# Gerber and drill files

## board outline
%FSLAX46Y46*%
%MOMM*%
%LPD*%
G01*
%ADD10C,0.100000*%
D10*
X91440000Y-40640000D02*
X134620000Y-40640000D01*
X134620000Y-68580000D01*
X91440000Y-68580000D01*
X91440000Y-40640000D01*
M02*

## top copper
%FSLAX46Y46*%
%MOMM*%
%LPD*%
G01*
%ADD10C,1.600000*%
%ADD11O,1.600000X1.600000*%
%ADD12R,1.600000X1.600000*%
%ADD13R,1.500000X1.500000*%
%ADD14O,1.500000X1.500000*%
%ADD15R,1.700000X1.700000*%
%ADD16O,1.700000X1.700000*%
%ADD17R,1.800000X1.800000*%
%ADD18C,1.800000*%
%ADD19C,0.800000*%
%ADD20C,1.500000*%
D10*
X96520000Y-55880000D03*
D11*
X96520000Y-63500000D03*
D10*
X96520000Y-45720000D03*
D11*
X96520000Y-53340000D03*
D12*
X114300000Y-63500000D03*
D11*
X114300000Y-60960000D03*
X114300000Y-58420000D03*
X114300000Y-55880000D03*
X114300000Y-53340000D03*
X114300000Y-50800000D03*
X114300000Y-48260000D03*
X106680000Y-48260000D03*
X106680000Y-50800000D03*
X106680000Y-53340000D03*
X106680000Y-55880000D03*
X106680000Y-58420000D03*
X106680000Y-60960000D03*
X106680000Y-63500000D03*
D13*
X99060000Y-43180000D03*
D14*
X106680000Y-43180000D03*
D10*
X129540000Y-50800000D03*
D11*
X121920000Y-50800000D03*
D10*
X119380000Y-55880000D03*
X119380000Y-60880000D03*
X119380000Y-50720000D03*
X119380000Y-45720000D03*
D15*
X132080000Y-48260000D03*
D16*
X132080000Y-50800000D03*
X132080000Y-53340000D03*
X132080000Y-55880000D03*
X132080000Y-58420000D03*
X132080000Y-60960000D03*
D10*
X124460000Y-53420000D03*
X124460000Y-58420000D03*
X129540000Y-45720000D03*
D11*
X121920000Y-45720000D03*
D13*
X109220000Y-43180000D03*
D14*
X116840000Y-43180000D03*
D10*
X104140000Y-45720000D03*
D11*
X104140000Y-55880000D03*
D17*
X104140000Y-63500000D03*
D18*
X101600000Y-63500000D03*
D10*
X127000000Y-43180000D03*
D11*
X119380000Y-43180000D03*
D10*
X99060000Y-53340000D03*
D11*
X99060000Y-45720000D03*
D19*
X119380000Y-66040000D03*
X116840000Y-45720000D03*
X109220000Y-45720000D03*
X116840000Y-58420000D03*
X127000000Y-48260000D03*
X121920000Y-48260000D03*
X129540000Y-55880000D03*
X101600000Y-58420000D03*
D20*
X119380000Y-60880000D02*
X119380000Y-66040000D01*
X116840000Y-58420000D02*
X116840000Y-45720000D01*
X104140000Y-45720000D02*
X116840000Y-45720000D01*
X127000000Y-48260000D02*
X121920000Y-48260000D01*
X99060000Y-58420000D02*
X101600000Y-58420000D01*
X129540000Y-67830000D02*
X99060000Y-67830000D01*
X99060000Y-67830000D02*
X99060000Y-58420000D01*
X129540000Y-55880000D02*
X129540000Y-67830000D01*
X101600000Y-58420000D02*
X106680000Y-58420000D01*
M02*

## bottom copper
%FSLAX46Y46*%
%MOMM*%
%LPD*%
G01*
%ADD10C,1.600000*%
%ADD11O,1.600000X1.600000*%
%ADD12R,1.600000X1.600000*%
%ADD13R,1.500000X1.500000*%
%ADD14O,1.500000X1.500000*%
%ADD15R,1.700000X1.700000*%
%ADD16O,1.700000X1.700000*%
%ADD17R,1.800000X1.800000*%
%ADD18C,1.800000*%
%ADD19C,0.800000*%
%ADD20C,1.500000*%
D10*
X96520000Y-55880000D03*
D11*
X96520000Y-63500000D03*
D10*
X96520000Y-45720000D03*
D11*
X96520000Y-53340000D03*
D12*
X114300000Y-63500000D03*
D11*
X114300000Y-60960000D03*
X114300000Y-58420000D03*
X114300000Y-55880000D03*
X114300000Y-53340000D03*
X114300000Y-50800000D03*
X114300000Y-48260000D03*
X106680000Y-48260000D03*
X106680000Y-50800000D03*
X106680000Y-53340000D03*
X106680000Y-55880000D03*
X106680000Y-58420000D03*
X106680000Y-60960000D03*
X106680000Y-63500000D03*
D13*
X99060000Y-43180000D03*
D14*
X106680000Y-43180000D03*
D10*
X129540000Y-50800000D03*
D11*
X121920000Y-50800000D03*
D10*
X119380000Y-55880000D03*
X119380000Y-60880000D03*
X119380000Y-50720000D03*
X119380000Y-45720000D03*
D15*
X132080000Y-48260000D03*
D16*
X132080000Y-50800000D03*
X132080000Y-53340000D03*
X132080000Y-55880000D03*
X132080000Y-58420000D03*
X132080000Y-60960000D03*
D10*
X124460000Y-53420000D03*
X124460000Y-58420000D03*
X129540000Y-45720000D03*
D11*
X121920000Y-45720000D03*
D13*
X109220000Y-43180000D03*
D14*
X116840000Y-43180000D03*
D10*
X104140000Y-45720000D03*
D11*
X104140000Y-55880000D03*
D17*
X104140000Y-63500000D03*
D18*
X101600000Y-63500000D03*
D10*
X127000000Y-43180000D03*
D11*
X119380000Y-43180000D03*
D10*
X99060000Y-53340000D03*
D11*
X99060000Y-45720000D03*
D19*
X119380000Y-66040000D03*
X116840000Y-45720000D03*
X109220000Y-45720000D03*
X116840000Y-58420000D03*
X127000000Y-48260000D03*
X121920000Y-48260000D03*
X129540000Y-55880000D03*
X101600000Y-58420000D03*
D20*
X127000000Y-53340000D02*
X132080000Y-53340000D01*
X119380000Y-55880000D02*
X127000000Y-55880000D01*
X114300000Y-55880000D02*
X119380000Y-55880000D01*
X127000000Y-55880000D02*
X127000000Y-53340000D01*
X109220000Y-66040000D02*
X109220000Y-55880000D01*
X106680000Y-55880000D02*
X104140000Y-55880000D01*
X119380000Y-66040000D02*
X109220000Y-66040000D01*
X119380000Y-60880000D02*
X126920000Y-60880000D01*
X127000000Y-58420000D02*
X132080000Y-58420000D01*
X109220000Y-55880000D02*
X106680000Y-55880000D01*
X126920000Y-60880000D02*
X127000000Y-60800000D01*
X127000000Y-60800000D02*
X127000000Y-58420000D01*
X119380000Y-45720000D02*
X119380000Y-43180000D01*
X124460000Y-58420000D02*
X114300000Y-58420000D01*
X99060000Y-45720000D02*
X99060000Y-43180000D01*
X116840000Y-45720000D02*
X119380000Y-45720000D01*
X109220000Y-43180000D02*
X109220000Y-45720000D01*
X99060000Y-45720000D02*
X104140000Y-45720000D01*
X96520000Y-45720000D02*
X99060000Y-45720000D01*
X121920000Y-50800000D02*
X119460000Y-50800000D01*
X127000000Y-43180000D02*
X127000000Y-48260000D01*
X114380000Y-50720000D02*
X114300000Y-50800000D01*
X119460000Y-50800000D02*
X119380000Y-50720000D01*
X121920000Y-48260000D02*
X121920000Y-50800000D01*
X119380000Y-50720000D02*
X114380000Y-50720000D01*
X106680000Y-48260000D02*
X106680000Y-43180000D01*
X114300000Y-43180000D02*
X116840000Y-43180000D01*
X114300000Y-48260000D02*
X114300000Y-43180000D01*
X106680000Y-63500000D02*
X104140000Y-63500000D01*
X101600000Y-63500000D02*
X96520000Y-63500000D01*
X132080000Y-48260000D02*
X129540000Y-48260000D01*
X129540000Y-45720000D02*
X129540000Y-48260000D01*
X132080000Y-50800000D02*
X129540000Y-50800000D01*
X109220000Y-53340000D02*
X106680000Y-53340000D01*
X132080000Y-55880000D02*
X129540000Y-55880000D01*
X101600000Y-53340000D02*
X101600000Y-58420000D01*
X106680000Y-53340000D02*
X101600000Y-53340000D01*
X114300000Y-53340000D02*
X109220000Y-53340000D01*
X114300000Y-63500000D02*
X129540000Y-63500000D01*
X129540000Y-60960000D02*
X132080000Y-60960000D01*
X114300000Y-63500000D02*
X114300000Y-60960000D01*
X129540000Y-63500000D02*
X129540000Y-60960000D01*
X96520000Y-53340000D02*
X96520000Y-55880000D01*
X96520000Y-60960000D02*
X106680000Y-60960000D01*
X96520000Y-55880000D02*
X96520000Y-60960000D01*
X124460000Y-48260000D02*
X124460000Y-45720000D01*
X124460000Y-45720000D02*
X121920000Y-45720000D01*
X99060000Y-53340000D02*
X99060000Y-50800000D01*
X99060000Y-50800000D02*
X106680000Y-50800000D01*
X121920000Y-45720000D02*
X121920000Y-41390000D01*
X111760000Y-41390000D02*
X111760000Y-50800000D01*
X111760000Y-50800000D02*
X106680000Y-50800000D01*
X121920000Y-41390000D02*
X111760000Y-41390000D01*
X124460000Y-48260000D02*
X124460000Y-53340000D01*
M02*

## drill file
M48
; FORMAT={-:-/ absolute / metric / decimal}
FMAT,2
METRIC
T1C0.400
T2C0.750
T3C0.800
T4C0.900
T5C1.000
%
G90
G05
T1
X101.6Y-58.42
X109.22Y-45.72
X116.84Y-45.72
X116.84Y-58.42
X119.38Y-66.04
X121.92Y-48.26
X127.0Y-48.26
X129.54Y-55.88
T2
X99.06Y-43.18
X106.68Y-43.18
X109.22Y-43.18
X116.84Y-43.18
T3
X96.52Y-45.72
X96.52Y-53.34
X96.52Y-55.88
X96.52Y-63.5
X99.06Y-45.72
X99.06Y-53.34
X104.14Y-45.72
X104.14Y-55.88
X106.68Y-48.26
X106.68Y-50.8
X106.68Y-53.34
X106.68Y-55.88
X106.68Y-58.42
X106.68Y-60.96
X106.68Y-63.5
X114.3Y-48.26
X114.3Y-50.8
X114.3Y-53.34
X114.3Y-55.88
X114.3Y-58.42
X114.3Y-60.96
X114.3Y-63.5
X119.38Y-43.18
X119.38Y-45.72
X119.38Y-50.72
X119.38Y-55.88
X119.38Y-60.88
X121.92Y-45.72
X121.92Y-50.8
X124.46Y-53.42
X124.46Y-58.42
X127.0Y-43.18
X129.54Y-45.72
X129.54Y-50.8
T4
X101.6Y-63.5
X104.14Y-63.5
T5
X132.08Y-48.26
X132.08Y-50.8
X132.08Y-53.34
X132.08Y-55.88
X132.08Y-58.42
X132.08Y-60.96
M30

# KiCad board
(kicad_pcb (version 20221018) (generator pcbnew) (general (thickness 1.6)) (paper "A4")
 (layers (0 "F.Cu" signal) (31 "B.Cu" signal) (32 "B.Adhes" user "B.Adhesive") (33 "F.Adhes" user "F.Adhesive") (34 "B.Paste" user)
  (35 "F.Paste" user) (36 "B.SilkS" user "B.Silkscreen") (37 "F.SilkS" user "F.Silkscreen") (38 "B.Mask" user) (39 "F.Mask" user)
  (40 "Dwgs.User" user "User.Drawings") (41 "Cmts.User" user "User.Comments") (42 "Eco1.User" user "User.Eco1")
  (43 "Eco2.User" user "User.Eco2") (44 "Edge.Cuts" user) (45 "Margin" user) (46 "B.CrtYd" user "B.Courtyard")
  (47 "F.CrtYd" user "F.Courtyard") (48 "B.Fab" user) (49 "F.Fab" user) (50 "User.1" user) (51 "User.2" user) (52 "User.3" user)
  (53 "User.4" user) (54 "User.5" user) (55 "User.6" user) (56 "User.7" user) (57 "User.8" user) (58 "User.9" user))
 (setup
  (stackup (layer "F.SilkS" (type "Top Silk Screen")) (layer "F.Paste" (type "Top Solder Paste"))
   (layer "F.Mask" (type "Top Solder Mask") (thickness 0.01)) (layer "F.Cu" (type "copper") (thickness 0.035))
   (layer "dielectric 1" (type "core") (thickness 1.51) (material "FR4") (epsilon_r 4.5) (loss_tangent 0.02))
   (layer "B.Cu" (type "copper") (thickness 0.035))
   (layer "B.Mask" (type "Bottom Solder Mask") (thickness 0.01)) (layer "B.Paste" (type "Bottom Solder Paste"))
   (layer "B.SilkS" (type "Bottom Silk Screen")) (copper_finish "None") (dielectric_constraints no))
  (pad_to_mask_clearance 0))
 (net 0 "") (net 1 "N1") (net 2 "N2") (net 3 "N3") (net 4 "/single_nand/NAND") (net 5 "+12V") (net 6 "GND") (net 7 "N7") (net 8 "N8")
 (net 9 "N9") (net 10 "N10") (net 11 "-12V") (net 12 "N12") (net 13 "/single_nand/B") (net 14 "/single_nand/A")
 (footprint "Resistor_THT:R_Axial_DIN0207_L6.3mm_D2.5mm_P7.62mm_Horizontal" (layer "F.Cu") (at 96.52 55.88 -90)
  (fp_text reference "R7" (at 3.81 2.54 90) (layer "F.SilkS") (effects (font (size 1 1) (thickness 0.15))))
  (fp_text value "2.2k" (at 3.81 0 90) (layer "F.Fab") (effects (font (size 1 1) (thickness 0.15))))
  (pad "1" thru_hole circle (at 0 0 270) (size 1.6 1.6) (drill 0.8) (layers "*.Cu" "*.Mask") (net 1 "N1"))
  (pad "2" thru_hole oval (at 7.62 0 270) (size 1.6 1.6) (drill 0.8) (layers "*.Cu" "*.Mask") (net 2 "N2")))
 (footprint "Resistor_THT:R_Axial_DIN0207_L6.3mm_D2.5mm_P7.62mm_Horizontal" (layer "F.Cu") (at 96.52 45.72 -90)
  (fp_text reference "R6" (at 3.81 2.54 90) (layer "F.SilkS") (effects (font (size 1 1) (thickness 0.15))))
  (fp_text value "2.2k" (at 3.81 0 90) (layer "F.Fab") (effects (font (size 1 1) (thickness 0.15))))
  (pad "1" thru_hole circle (at 0 0 270) (size 1.6 1.6) (drill 0.8) (layers "*.Cu" "*.Mask") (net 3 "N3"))
  (pad "2" thru_hole oval (at 7.62 0 270) (size 1.6 1.6) (drill 0.8) (layers "*.Cu" "*.Mask") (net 1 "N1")))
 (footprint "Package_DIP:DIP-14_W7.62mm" (layer "F.Cu") (at 114.3 63.5 180)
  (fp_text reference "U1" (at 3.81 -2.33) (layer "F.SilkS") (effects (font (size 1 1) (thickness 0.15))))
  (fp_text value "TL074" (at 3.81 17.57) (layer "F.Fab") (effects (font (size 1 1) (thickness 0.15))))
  (pad "1" thru_hole rect (at 0 0 180) (size 1.6 1.6) (drill 0.8) (layers "*.Cu" "*.Mask") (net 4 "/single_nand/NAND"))
  (pad "2" thru_hole oval (at 0 2.54 180) (size 1.6 1.6) (drill 0.8) (layers "*.Cu" "*.Mask") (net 4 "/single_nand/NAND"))
  (pad "3" thru_hole oval (at 0 5.08 180) (size 1.6 1.6) (drill 0.8) (layers "*.Cu" "*.Mask") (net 3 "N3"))
  (pad "4" thru_hole oval (at 0 7.62 180) (size 1.6 1.6) (drill 0.8) (layers "*.Cu" "*.Mask") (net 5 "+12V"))
  (pad "5" thru_hole oval (at 0 10.16 180) (size 1.6 1.6) (drill 0.8) (layers "*.Cu" "*.Mask") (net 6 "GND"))
  (pad "6" thru_hole oval (at 0 12.7 180) (size 1.6 1.6) (drill 0.8) (layers "*.Cu" "*.Mask") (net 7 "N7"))
  (pad "7" thru_hole oval (at 0 15.24 180) (size 1.6 1.6) (drill 0.8) (layers "*.Cu" "*.Mask") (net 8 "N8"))
  (pad "8" thru_hole oval (at 7.62 15.24 180) (size 1.6 1.6) (drill 0.8) (layers "*.Cu" "*.Mask") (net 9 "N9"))
  (pad "9" thru_hole oval (at 7.62 12.7 180) (size 1.6 1.6) (drill 0.8) (layers "*.Cu" "*.Mask") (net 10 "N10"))
  (pad "10" thru_hole oval (at 7.62 10.16 180) (size 1.6 1.6) (drill 0.8) (layers "*.Cu" "*.Mask") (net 6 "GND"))
  (pad "11" thru_hole oval (at 7.62 7.62 180) (size 1.6 1.6) (drill 0.8) (layers "*.Cu" "*.Mask") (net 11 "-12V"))
  (pad "12" thru_hole oval (at 7.62 5.08 180) (size 1.6 1.6) (drill 0.8) (layers "*.Cu" "*.Mask") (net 6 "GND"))
  (pad "13" thru_hole oval (at 7.62 2.54 180) (size 1.6 1.6) (drill 0.8) (layers "*.Cu" "*.Mask") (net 1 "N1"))
  (pad "14" thru_hole oval (at 7.62 0 180) (size 1.6 1.6) (drill 0.8) (layers "*.Cu" "*.Mask") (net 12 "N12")))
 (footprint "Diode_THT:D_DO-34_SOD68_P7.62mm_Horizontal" (layer "F.Cu") (at 99.06 43.18)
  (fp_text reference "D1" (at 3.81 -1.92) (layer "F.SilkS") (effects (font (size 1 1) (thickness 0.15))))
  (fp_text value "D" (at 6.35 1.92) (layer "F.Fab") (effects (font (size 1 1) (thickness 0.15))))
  (pad "1" thru_hole rect (at 0 0) (size 1.5 1.5) (drill 0.75) (layers "*.Cu" "*.Mask") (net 3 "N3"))
  (pad "2" thru_hole oval (at 7.62 0) (size 1.5 1.5) (drill 0.75) (layers "*.Cu" "*.Mask") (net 9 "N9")))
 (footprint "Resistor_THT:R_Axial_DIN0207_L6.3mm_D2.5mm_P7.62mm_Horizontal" (layer "F.Cu") (at 129.54 50.8 180)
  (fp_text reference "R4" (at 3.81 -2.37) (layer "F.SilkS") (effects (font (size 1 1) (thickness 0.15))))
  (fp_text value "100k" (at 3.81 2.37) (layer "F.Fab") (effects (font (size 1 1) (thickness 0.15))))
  (pad "1" thru_hole circle (at 0 0 180) (size 1.6 1.6) (drill 0.8) (layers "*.Cu" "*.Mask") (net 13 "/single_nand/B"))
  (pad "2" thru_hole oval (at 7.62 0 180) (size 1.6 1.6) (drill 0.8) (layers "*.Cu" "*.Mask") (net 7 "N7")))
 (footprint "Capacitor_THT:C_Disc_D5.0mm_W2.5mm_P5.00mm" (layer "F.Cu") (at 119.38 55.88 -90)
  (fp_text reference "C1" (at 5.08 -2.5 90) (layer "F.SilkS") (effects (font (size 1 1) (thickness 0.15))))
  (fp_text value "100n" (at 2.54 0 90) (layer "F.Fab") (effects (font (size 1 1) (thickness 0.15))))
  (pad "1" thru_hole circle (at 0 0 270) (size 1.6 1.6) (drill 0.8) (layers "*.Cu" "*.Mask") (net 5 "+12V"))
  (pad "2" thru_hole circle (at 5 0 270) (size 1.6 1.6) (drill 0.8) (layers "*.Cu" "*.Mask") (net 11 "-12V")))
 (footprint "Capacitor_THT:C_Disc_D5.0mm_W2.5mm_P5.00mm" (layer "F.Cu") (at 119.38 50.72 90)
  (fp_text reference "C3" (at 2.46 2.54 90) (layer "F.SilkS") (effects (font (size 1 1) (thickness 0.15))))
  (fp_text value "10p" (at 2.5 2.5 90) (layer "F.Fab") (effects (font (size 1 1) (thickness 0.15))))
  (pad "1" thru_hole circle (at 0 0 90) (size 1.6 1.6) (drill 0.8) (layers "*.Cu" "*.Mask") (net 7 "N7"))
  (pad "2" thru_hole circle (at 5 0 90) (size 1.6 1.6) (drill 0.8) (layers "*.Cu" "*.Mask") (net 3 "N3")))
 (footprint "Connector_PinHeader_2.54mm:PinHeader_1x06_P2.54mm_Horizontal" (layer "F.Cu") (at 132.08 48.26)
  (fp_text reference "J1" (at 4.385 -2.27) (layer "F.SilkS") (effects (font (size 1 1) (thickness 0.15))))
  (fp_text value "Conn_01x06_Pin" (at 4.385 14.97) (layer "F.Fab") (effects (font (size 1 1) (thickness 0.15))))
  (pad "1" thru_hole rect (at 0 0) (size 1.7 1.7) (drill 1) (layers "*.Cu" "*.Mask") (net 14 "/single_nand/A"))
  (pad "2" thru_hole oval (at 0 2.54) (size 1.7 1.7) (drill 1) (layers "*.Cu" "*.Mask") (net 13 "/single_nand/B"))
  (pad "3" thru_hole oval (at 0 5.08) (size 1.7 1.7) (drill 1) (layers "*.Cu" "*.Mask") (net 5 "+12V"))
  (pad "4" thru_hole oval (at 0 7.62) (size 1.7 1.7) (drill 1) (layers "*.Cu" "*.Mask") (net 6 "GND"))
  (pad "5" thru_hole oval (at 0 10.16) (size 1.7 1.7) (drill 1) (layers "*.Cu" "*.Mask") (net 11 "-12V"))
  (pad "6" thru_hole oval (at 0 12.7) (size 1.7 1.7) (drill 1) (layers "*.Cu" "*.Mask") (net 4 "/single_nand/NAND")))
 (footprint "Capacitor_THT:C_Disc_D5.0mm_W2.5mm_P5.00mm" (layer "F.Cu") (at 124.46 53.42 -90)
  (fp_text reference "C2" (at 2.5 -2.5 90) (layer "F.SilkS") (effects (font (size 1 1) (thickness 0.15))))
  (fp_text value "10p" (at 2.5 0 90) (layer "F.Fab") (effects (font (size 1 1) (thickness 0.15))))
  (pad "1" thru_hole circle (at 0 0 270) (size 1.6 1.6) (drill 0.8) (layers "*.Cu" "*.Mask") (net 10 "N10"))
  (pad "2" thru_hole circle (at 5 0 270) (size 1.6 1.6) (drill 0.8) (layers "*.Cu" "*.Mask") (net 3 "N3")))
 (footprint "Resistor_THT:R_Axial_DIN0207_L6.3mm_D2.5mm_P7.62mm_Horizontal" (layer "F.Cu") (at 129.54 45.72 180)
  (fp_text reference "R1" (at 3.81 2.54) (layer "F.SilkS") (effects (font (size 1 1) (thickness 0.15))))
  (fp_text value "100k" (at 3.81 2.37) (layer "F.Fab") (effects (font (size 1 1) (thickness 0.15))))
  (pad "1" thru_hole circle (at 0 0 180) (size 1.6 1.6) (drill 0.8) (layers "*.Cu" "*.Mask") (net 14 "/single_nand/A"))
  (pad "2" thru_hole oval (at 7.62 0 180) (size 1.6 1.6) (drill 0.8) (layers "*.Cu" "*.Mask") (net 10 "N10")))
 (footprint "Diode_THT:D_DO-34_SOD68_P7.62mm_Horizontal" (layer "F.Cu") (at 109.22 43.18)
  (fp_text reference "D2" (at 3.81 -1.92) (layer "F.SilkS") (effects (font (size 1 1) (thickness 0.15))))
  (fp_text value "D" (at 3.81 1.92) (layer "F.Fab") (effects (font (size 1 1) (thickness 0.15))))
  (pad "1" thru_hole rect (at 0 0) (size 1.5 1.5) (drill 0.75) (layers "*.Cu" "*.Mask") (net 3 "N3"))
  (pad "2" thru_hole oval (at 7.62 0) (size 1.5 1.5) (drill 0.75) (layers "*.Cu" "*.Mask") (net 8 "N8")))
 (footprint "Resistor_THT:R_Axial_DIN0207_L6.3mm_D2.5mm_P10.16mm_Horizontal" (layer "F.Cu") (at 104.14 45.72 -90)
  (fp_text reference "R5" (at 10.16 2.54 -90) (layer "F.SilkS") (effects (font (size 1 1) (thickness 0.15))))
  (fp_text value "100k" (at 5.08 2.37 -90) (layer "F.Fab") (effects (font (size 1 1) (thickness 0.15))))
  (pad "1" thru_hole circle (at 0 0 270) (size 1.6 1.6) (drill 0.8) (layers "*.Cu" "*.Mask") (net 3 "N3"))
  (pad "2" thru_hole oval (at 10.16 0 270) (size 1.6 1.6) (drill 0.8) (layers "*.Cu" "*.Mask") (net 11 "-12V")))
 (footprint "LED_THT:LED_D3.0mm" (layer "F.Cu") (at 104.14 63.5 180)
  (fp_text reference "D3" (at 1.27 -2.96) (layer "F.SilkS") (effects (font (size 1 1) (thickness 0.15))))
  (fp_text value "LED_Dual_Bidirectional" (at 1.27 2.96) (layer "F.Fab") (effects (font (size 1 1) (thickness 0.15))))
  (pad "1" thru_hole rect (at 0 0 180) (size 1.8 1.8) (drill 0.9) (layers "*.Cu" "*.Mask") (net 12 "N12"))
  (pad "2" thru_hole circle (at 2.54 0 180) (size 1.8 1.8) (drill 0.9) (layers "*.Cu" "*.Mask") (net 2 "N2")))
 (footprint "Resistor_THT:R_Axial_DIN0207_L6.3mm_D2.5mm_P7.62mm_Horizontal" (layer "F.Cu") (at 127 43.18 180)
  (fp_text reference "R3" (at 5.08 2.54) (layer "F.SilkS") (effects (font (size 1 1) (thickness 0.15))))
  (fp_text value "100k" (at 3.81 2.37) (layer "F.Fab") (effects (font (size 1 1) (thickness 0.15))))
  (pad "1" thru_hole circle (at 0 0 180) (size 1.6 1.6) (drill 0.8) (layers "*.Cu" "*.Mask") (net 7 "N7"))
  (pad "2" thru_hole oval (at 7.62 0 180) (size 1.6 1.6) (drill 0.8) (layers "*.Cu" "*.Mask") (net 3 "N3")))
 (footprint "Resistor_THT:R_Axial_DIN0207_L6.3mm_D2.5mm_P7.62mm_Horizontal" (layer "F.Cu") (at 99.06 53.34 90)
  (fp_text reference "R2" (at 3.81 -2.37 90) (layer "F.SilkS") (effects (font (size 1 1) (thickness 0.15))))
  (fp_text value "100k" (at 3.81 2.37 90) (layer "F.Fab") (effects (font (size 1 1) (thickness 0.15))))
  (pad "1" thru_hole circle (at 0 0 90) (size 1.6 1.6) (drill 0.8) (layers "*.Cu" "*.Mask") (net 10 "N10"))
  (pad "2" thru_hole oval (at 7.62 0 90) (size 1.6 1.6) (drill 0.8) (layers "*.Cu" "*.Mask") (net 3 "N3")))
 (gr_rect (start 91.44 40.64) (end 134.62 68.58) (stroke (width 0.1) (type default)) (fill none) (layer "Edge.Cuts"))
 (segment (start 127 53.34) (end 132.08 53.34) (width 1.5) (layer "B.Cu") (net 5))
 (segment (start 119.38 55.88) (end 127 55.88) (width 1.5) (layer "B.Cu") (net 5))
 (segment (start 114.3 55.88) (end 119.38 55.88) (width 1.5) (layer "B.Cu") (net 5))
 (segment (start 127 55.88) (end 127 53.34) (width 1.5) (layer "B.Cu") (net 5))
 (segment (start 119.38 60.88) (end 119.38 66.04) (width 1.5) (layer "F.Cu") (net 11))
 (via (at 119.38 66.04) (size 0.8) (drill 0.4) (layers "F.Cu" "B.Cu") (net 11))
 (segment (start 109.22 66.04) (end 109.22 55.88) (width 1.5) (layer "B.Cu") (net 11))
 (segment (start 106.68 55.88) (end 104.14 55.88) (width 1.5) (layer "B.Cu") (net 11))
 (segment (start 119.38 66.04) (end 109.22 66.04) (width 1.5) (layer "B.Cu") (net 11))
 (segment (start 119.38 60.88) (end 126.92 60.88) (width 1.5) (layer "B.Cu") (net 11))
 (segment (start 127 58.42) (end 132.08 58.42) (width 1.5) (layer "B.Cu") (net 11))
 (segment (start 109.22 55.88) (end 106.68 55.88) (width 1.5) (layer "B.Cu") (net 11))
 (segment (start 126.92 60.88) (end 127 60.8) (width 1.5) (layer "B.Cu") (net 11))
 (segment (start 127 60.8) (end 127 58.42) (width 1.5) (layer "B.Cu") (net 11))
 (segment (start 116.84 58.42) (end 116.84 45.72) (width 1.5) (layer "F.Cu") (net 3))
 (segment (start 104.14 45.72) (end 116.84 45.72) (width 1.5) (layer "F.Cu") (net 3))
 (via (at 116.84 45.72) (size 0.8) (drill 0.4) (layers "F.Cu" "B.Cu") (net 3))
 (via (at 109.22 45.72) (size 0.8) (drill 0.4) (layers "F.Cu" "B.Cu") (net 3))
 (via (at 116.84 58.42) (size 0.8) (drill 0.4) (layers "F.Cu" "B.Cu") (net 3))
 (segment (start 119.38 45.72) (end 119.38 43.18) (width 1.5) (layer "B.Cu") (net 3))
 (segment (start 124.46 58.42) (end 114.3 58.42) (width 1.5) (layer "B.Cu") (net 3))
 (segment (start 99.06 45.72) (end 99.06 43.18) (width 1.5) (layer "B.Cu") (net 3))
 (segment (start 116.84 45.72) (end 119.38 45.72) (width 1.5) (layer "B.Cu") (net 3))
 (segment (start 109.22 43.18) (end 109.22 45.72) (width 1.5) (layer "B.Cu") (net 3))
 (segment (start 99.06 45.72) (end 104.14 45.72) (width 1.5) (layer "B.Cu") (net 3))
 (segment (start 96.52 45.72) (end 99.06 45.72) (width 1.5) (layer "B.Cu") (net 3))
 (segment (start 127 48.26) (end 121.92 48.26) (width 1.5) (layer "F.Cu") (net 7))
 (via (at 127 48.26) (size 0.8) (drill 0.4) (layers "F.Cu" "B.Cu") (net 7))
 (via (at 121.92 48.26) (size 0.8) (drill 0.4) (layers "F.Cu" "B.Cu") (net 7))
 (segment (start 121.92 50.8) (end 119.46 50.8) (width 1.5) (layer "B.Cu") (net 7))
 (segment (start 127 43.18) (end 127 48.26) (width 1.5) (layer "B.Cu") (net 7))
 (segment (start 114.38 50.72) (end 114.3 50.8) (width 1.5) (layer "B.Cu") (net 7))
 (segment (start 119.46 50.8) (end 119.38 50.72) (width 1.5) (layer "B.Cu") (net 7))
 (segment (start 121.92 48.26) (end 121.92 50.8) (width 1.5) (layer "B.Cu") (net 7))
 (segment (start 119.38 50.72) (end 114.38 50.72) (width 1.5) (layer "B.Cu") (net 7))
 (segment (start 106.68 48.26) (end 106.68 43.18) (width 1.5) (layer "B.Cu") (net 9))
 (segment (start 114.3 43.18) (end 116.84 43.18) (width 1.5) (layer "B.Cu") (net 8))
 (segment (start 114.3 48.26) (end 114.3 43.18) (width 1.5) (layer "B.Cu") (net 8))
 (segment (start 106.68 63.5) (end 104.14 63.5) (width 1.5) (layer "B.Cu") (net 12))
 (segment (start 101.6 63.5) (end 96.52 63.5) (width 1.5) (layer "B.Cu") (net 2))
 (segment (start 132.08 48.26) (end 129.54 48.26) (width 1.5) (layer "B.Cu") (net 14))
 (segment (start 129.54 45.72) (end 129.54 48.26) (width 1.5) (layer "B.Cu") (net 14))
 (segment (start 132.08 50.8) (end 129.54 50.8) (width 1.5) (layer "B.Cu") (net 13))
 (segment (start 99.06 58.42) (end 101.6 58.42) (width 1.5) (layer "F.Cu") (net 6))
 (segment (start 129.54 67.83) (end 99.06 67.83) (width 1.5) (layer "F.Cu") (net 6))
 (segment (start 99.06 67.83) (end 99.06 58.42) (width 1.5) (layer "F.Cu") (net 6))
 (segment (start 129.54 55.88) (end 129.54 67.83) (width 1.5) (layer "F.Cu") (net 6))
 (segment (start 101.6 58.42) (end 106.68 58.42) (width 1.5) (layer "F.Cu") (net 6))
 (via (at 129.54 55.88) (size 0.8) (drill 0.4) (layers "F.Cu" "B.Cu") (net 6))
 (via (at 101.6 58.42) (size 0.8) (drill 0.4) (layers "F.Cu" "B.Cu") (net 6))
 (segment (start 109.22 53.34) (end 106.68 53.34) (width 1.5) (layer "B.Cu") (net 6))
 (segment (start 132.08 55.88) (end 129.54 55.88) (width 1.5) (layer "B.Cu") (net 6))
 (segment (start 101.6 53.34) (end 101.6 58.42) (width 1.5) (layer "B.Cu") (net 6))
 (segment (start 106.68 53.34) (end 101.6 53.34) (width 1.5) (layer "B.Cu") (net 6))
 (segment (start 114.3 53.34) (end 109.22 53.34) (width 1.5) (layer "B.Cu") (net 6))
 (segment (start 114.3 63.5) (end 129.54 63.5) (width 1.5) (layer "B.Cu") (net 4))
 (segment (start 129.54 60.96) (end 132.08 60.96) (width 1.5) (layer "B.Cu") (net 4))
 (segment (start 114.3 63.5) (end 114.3 60.96) (width 1.5) (layer "B.Cu") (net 4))
 (segment (start 129.54 63.5) (end 129.54 60.96) (width 1.5) (layer "B.Cu") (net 4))
 (segment (start 96.52 53.34) (end 96.52 55.88) (width 1.5) (layer "B.Cu") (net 1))
 (segment (start 96.52 60.96) (end 106.68 60.96) (width 1.5) (layer "B.Cu") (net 1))
 (segment (start 96.52 55.88) (end 96.52 60.96) (width 1.5) (layer "B.Cu") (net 1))
 (segment (start 124.46 48.26) (end 124.46 45.72) (width 1.5) (layer "B.Cu") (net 10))
 (segment (start 124.46 45.72) (end 121.92 45.72) (width 1.5) (layer "B.Cu") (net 10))
 (segment (start 99.06 53.34) (end 99.06 50.8) (width 1.5) (layer "B.Cu") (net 10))
 (segment (start 99.06 50.8) (end 106.68 50.8) (width 1.5) (layer "B.Cu") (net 10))
 (segment (start 121.92 45.72) (end 121.92 41.39) (width 1.5) (layer "B.Cu") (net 10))
 (segment (start 111.76 41.39) (end 111.76 50.8) (width 1.5) (layer "B.Cu") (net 10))
 (segment (start 111.76 50.8) (end 106.68 50.8) (width 1.5) (layer "B.Cu") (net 10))
 (segment (start 121.92 41.39) (end 111.76 41.39) (width 1.5) (layer "B.Cu") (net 10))
 (segment (start 124.46 48.26) (end 124.46 53.34) (width 1.5) (layer "B.Cu") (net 10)))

